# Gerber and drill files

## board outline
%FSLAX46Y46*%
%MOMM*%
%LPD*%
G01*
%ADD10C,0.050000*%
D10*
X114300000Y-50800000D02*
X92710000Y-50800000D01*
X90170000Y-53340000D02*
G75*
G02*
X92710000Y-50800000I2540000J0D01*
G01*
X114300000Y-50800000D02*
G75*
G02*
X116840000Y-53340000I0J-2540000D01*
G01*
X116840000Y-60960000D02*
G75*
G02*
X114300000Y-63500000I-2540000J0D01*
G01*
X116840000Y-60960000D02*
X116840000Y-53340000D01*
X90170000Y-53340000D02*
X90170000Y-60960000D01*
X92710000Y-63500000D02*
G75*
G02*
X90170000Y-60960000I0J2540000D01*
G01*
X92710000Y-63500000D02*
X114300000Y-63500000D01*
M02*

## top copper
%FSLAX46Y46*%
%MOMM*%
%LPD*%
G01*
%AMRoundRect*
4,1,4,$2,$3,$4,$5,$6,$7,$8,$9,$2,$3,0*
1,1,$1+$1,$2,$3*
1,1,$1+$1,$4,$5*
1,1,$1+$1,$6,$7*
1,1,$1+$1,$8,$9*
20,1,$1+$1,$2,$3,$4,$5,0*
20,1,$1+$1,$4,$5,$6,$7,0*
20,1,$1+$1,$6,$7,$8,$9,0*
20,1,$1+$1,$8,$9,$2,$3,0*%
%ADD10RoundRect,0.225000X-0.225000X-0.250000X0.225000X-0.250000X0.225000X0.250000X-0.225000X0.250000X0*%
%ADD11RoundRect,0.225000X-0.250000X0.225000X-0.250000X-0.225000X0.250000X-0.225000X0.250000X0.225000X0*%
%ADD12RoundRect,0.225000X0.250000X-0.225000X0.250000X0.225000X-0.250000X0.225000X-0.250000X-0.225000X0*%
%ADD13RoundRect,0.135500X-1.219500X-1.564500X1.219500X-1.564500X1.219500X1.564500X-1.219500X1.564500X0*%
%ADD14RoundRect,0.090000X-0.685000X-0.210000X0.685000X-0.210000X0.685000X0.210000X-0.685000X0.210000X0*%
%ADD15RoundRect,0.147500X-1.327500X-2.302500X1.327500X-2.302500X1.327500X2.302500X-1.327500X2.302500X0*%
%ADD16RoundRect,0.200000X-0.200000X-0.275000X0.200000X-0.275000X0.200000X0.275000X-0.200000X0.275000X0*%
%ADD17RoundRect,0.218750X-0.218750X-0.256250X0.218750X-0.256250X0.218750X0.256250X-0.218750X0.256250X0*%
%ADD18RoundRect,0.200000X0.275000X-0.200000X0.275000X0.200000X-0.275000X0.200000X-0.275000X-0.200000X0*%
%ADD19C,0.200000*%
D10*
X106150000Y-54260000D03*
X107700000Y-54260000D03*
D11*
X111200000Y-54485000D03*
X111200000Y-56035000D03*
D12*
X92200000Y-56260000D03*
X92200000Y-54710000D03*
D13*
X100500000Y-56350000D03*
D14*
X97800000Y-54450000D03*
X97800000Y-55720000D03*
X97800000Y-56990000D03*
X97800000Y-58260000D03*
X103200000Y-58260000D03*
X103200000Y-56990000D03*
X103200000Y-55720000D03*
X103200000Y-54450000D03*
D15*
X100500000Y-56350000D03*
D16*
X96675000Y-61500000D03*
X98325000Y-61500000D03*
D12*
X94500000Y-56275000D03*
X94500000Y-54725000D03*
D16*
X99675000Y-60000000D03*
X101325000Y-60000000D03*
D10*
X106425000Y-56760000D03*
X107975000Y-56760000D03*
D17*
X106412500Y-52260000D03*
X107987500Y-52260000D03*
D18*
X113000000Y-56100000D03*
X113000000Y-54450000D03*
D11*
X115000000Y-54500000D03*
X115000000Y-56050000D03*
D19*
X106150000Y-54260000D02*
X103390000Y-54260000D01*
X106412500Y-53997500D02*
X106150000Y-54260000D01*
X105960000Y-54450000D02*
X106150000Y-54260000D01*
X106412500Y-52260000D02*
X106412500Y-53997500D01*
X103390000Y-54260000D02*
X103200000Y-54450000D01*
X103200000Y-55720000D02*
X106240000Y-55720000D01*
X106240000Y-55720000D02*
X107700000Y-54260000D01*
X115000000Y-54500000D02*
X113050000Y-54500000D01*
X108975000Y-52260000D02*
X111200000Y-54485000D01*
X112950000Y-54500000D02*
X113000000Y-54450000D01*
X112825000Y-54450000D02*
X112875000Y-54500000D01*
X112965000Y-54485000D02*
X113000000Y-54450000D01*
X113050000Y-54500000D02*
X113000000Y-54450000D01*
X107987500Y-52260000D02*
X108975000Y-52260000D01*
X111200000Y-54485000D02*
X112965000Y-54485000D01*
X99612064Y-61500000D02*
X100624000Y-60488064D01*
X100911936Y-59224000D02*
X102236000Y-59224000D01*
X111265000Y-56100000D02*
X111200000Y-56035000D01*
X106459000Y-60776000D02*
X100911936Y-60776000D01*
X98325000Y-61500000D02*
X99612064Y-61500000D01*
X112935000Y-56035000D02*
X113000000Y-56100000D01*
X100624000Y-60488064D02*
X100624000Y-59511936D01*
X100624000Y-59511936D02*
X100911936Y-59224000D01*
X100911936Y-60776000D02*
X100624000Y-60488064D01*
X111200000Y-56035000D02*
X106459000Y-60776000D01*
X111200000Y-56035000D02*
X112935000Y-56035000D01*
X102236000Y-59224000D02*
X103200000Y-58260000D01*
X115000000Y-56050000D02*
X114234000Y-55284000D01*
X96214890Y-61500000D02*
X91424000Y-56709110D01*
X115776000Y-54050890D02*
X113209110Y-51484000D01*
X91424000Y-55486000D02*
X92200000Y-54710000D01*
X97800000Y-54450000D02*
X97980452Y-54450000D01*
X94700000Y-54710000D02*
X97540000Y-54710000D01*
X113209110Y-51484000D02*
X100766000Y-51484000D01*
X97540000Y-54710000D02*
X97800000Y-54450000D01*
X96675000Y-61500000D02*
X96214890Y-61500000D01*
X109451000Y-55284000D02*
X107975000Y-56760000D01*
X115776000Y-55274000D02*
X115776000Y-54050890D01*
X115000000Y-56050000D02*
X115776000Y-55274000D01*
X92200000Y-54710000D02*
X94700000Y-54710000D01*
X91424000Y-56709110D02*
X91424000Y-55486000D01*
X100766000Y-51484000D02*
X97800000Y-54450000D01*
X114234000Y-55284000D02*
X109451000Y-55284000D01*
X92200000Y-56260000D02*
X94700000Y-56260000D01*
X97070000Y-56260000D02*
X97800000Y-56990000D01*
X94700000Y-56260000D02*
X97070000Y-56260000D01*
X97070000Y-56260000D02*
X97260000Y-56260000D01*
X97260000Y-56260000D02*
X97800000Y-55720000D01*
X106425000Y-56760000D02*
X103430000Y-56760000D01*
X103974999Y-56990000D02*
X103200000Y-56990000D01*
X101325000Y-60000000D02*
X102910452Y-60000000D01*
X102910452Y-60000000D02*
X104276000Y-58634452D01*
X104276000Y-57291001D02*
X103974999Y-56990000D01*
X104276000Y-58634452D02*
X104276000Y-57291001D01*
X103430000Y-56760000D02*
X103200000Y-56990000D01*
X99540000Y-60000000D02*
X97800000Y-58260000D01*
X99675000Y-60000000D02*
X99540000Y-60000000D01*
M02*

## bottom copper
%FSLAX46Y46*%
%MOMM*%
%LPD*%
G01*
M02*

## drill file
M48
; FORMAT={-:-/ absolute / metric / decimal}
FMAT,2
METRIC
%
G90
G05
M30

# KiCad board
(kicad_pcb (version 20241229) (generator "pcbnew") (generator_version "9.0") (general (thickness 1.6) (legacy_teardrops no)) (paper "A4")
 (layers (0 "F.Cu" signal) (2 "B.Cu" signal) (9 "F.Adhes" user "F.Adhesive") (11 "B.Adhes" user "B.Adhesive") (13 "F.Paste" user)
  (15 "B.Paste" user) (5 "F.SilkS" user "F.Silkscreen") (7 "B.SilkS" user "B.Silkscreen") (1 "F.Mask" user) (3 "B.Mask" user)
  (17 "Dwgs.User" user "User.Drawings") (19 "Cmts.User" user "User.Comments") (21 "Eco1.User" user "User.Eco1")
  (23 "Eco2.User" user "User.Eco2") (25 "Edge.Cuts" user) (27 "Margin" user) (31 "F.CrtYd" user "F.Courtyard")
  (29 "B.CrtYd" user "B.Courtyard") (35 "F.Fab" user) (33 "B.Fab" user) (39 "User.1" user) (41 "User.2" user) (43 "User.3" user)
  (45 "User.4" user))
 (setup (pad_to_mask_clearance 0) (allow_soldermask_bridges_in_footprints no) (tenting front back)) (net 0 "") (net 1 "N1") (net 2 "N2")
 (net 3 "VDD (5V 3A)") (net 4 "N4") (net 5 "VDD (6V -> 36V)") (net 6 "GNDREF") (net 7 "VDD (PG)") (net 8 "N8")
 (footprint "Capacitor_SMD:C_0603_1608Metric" (layer "F.Cu") (at 106.925 54.26)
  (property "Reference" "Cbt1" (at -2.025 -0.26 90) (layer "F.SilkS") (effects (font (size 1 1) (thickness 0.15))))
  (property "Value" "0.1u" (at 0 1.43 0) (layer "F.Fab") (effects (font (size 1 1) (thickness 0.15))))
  (pad "1" smd roundrect (at -0.775 0) (size 0.9 0.95) (layers "F.Cu" "F.Mask" "F.Paste") (roundrect_rratio 0.25) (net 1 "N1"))
  (pad "2" smd roundrect (at 0.775 0) (size 0.9 0.95) (layers "F.Cu" "F.Mask" "F.Paste") (roundrect_rratio 0.25) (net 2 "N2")))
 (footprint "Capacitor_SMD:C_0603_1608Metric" (layer "F.Cu") (at 111.2 55.26 -90)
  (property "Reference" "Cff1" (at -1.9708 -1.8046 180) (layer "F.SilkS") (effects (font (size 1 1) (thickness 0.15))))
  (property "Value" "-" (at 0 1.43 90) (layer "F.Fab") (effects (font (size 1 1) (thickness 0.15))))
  (pad "1" smd roundrect (at -0.775 0 270) (size 0.9 0.95) (layers "F.Cu" "F.Mask" "F.Paste") (roundrect_rratio 0.25) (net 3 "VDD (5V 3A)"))
  (pad "2" smd roundrect (at 0.775 0 270) (size 0.9 0.95) (layers "F.Cu" "F.Mask" "F.Paste") (roundrect_rratio 0.25) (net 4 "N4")))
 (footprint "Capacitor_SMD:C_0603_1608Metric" (layer "F.Cu") (at 92.2 55.485 90)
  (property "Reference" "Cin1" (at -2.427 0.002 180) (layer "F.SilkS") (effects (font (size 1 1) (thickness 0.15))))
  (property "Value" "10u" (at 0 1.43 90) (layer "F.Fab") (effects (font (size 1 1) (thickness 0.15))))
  (pad "1" smd roundrect (at -0.775 0 90) (size 0.9 0.95) (layers "F.Cu" "F.Mask" "F.Paste") (roundrect_rratio 0.25)
   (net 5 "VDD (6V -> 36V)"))
  (pad "2" smd roundrect (at 0.775 0 90) (size 0.9 0.95) (layers "F.Cu" "F.Mask" "F.Paste") (roundrect_rratio 0.25) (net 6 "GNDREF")))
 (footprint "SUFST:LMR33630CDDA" (layer "F.Cu") (at 100.4 53.35)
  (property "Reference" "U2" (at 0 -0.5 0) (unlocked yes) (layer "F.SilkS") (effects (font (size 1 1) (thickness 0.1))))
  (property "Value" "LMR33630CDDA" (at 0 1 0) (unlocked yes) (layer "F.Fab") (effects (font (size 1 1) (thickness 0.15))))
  (pad "" smd roundrect (at 0.1 3) (size 2.71 3.4) (layers "F.Cu" "F.Mask" "F.Paste") (roundrect_rratio 0.05))
  (pad "1" smd roundrect (at -2.6 1.1) (size 1.55 0.6) (layers "F.Cu" "F.Mask" "F.Paste") (roundrect_rratio 0.15) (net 6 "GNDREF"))
  (pad "2" smd roundrect (at -2.6 2.37) (size 1.55 0.6) (layers "F.Cu" "F.Mask" "F.Paste") (roundrect_rratio 0.15) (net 5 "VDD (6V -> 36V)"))
  (pad "3" smd roundrect (at -2.6 3.64) (size 1.55 0.6) (layers "F.Cu" "F.Mask" "F.Paste") (roundrect_rratio 0.15) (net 5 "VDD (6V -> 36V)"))
  (pad "4" smd roundrect (at -2.6 4.91) (size 1.55 0.6) (layers "F.Cu" "F.Mask" "F.Paste") (roundrect_rratio 0.15) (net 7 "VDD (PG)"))
  (pad "5" smd roundrect (at 2.8 4.91) (size 1.55 0.6) (layers "F.Cu" "F.Mask" "F.Paste") (roundrect_rratio 0.15) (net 4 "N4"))
  (pad "6" smd roundrect (at 2.8 3.64) (size 1.55 0.6) (layers "F.Cu" "F.Mask" "F.Paste") (roundrect_rratio 0.15) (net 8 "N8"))
  (pad "7" smd roundrect (at 2.8 2.37) (size 1.55 0.6) (layers "F.Cu" "F.Mask" "F.Paste") (roundrect_rratio 0.15) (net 2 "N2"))
  (pad "8" smd roundrect (at 2.8 1.1) (size 1.55 0.6) (layers "F.Cu" "F.Mask" "F.Paste") (roundrect_rratio 0.15) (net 1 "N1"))
  (pad "TP" smd roundrect (at 0.1 3) (size 2.95 4.9) (layers "F.Cu") (roundrect_rratio 0.05) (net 6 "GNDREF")))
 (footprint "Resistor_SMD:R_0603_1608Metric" (layer "F.Cu") (at 97.5 61.5)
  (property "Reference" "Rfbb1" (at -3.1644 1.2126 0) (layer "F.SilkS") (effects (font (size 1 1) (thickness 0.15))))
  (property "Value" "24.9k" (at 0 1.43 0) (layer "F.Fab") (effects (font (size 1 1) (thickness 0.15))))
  (pad "1" smd roundrect (at -0.825 0) (size 0.8 0.95) (layers "F.Cu" "F.Mask" "F.Paste") (roundrect_rratio 0.25) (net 6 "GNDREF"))
  (pad "2" smd roundrect (at 0.825 0) (size 0.8 0.95) (layers "F.Cu" "F.Mask" "F.Paste") (roundrect_rratio 0.25) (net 4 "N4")))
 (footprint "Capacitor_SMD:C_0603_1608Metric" (layer "F.Cu") (at 94.5 55.5 90)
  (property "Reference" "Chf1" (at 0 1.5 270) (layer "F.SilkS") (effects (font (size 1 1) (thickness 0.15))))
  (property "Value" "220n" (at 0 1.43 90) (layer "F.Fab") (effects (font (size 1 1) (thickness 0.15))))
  (pad "1" smd roundrect (at -0.775 0 90) (size 0.9 0.95) (layers "F.Cu" "F.Mask" "F.Paste") (roundrect_rratio 0.25)
   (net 5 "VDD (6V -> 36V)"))
  (pad "2" smd roundrect (at 0.775 0 90) (size 0.9 0.95) (layers "F.Cu" "F.Mask" "F.Paste") (roundrect_rratio 0.25) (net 6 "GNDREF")))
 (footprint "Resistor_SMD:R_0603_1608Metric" (layer "F.Cu") (at 100.5 60)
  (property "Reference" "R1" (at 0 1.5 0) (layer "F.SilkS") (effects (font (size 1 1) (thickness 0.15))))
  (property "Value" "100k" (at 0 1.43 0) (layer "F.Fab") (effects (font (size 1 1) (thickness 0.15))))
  (pad "1" smd roundrect (at -0.825 0) (size 0.8 0.95) (layers "F.Cu" "F.Mask" "F.Paste") (roundrect_rratio 0.25) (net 7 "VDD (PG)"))
  (pad "2" smd roundrect (at 0.825 0) (size 0.8 0.95) (layers "F.Cu" "F.Mask" "F.Paste") (roundrect_rratio 0.25) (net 8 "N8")))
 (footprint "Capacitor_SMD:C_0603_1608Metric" (layer "F.Cu") (at 107.2 56.76)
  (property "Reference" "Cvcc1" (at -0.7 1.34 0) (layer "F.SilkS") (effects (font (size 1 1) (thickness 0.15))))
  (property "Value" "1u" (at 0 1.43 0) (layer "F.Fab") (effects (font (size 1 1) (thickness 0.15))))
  (pad "1" smd roundrect (at -0.775 0) (size 0.9 0.95) (layers "F.Cu" "F.Mask" "F.Paste") (roundrect_rratio 0.25) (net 8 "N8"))
  (pad "2" smd roundrect (at 0.775 0) (size 0.9 0.95) (layers "F.Cu" "F.Mask" "F.Paste") (roundrect_rratio 0.25) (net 6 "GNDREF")))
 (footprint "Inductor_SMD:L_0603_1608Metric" (layer "F.Cu") (at 107.2 52.26)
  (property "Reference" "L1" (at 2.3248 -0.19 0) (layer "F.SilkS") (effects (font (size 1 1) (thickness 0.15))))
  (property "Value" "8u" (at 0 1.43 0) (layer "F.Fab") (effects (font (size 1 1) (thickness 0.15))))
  (pad "1" smd roundrect (at -0.7875 0) (size 0.875 0.95) (layers "F.Cu" "F.Mask" "F.Paste") (roundrect_rratio 0.25) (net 1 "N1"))
  (pad "2" smd roundrect (at 0.7875 0) (size 0.875 0.95) (layers "F.Cu" "F.Mask" "F.Paste") (roundrect_rratio 0.25) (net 3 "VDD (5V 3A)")))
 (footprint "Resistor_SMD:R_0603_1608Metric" (layer "F.Cu") (at 113 55.275 90)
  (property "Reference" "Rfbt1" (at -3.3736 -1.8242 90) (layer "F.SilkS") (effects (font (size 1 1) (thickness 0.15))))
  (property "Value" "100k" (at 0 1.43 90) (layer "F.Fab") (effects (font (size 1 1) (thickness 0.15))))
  (pad "1" smd roundrect (at -0.825 0 90) (size 0.8 0.95) (layers "F.Cu" "F.Mask" "F.Paste") (roundrect_rratio 0.25) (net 4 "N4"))
  (pad "2" smd roundrect (at 0.825 0 90) (size 0.8 0.95) (layers "F.Cu" "F.Mask" "F.Paste") (roundrect_rratio 0.25) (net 3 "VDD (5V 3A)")))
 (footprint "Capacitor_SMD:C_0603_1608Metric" (layer "F.Cu") (at 115 55.275 -90)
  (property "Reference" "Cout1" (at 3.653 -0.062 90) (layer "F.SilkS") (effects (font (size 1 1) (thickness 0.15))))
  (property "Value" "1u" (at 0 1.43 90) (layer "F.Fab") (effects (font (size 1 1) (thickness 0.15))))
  (pad "1" smd roundrect (at -0.775 0 270) (size 0.9 0.95) (layers "F.Cu" "F.Mask" "F.Paste") (roundrect_rratio 0.25) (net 3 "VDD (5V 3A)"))
  (pad "2" smd roundrect (at 0.775 0 270) (size 0.9 0.95) (layers "F.Cu" "F.Mask" "F.Paste") (roundrect_rratio 0.25) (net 6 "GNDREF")))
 (gr_line (start 114.3 50.8) (end 92.71 50.8) (stroke (width 0.05) (type default)) (layer "Edge.Cuts"))
 (gr_arc (start 90.17 53.34) (mid 90.913949 51.543949) (end 92.71 50.8) (stroke (width 0.05) (type default)) (layer "Edge.Cuts"))
 (gr_arc (start 114.3 50.8) (mid 116.096051 51.543949) (end 116.84 53.34) (stroke (width 0.05) (type default)) (layer "Edge.Cuts"))
 (gr_arc (start 116.84 60.96) (mid 116.096051 62.756051) (end 114.3 63.5) (stroke (width 0.05) (type default)) (layer "Edge.Cuts"))
 (gr_line (start 116.84 60.96) (end 116.84 53.34) (stroke (width 0.05) (type default)) (layer "Edge.Cuts"))
 (gr_line (start 90.17 53.34) (end 90.17 60.96) (stroke (width 0.05) (type default)) (layer "Edge.Cuts"))
 (gr_arc (start 92.71 63.5) (mid 90.913949 62.756051) (end 90.17 60.96) (stroke (width 0.05) (type default)) (layer "Edge.Cuts"))
 (gr_line (start 92.71 63.5) (end 114.3 63.5) (stroke (width 0.05) (type default)) (layer "Edge.Cuts"))
 (segment (start 106.15 54.26) (end 103.39 54.26) (width 0.2) (layer "F.Cu") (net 1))
 (segment (start 106.4125 53.9975) (end 106.15 54.26) (width 0.2) (layer "F.Cu") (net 1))
 (segment (start 105.96 54.45) (end 106.15 54.26) (width 0.2) (layer "F.Cu") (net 1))
 (segment (start 106.4125 52.26) (end 106.4125 53.9975) (width 0.2) (layer "F.Cu") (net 1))
 (segment (start 103.39 54.26) (end 103.2 54.45) (width 0.2) (layer "F.Cu") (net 1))
 (segment (start 103.2 55.72) (end 106.24 55.72) (width 0.2) (layer "F.Cu") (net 2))
 (segment (start 106.24 55.72) (end 107.7 54.26) (width 0.2) (layer "F.Cu") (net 2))
 (segment (start 115 54.5) (end 113.05 54.5) (width 0.2) (layer "F.Cu") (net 3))
 (segment (start 108.975 52.26) (end 111.2 54.485) (width 0.2) (layer "F.Cu") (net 3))
 (segment (start 112.95 54.5) (end 113 54.45) (width 0.2) (layer "F.Cu") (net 3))
 (segment (start 112.825 54.45) (end 112.875 54.5) (width 0.2) (layer "F.Cu") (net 3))
 (segment (start 112.965 54.485) (end 113 54.45) (width 0.2) (layer "F.Cu") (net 3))
 (segment (start 113.05 54.5) (end 113 54.45) (width 0.2) (layer "F.Cu") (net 3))
 (segment (start 107.9875 52.26) (end 108.975 52.26) (width 0.2) (layer "F.Cu") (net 3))
 (segment (start 111.2 54.485) (end 112.965 54.485) (width 0.2) (layer "F.Cu") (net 3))
 (segment (start 99.612064 61.5) (end 100.624 60.488064) (width 0.2) (layer "F.Cu") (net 4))
 (segment (start 100.911936 59.224) (end 102.236 59.224) (width 0.2) (layer "F.Cu") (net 4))
 (segment (start 111.265 56.1) (end 111.2 56.035) (width 0.2) (layer "F.Cu") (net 4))
 (segment (start 106.459 60.776) (end 100.911936 60.776) (width 0.2) (layer "F.Cu") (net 4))
 (segment (start 98.325 61.5) (end 99.612064 61.5) (width 0.2) (layer "F.Cu") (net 4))
 (segment (start 112.935 56.035) (end 113 56.1) (width 0.2) (layer "F.Cu") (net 4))
 (segment (start 100.624 60.488064) (end 100.624 59.511936) (width 0.2) (layer "F.Cu") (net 4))
 (segment (start 100.624 59.511936) (end 100.911936 59.224) (width 0.2) (layer "F.Cu") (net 4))
 (segment (start 100.911936 60.776) (end 100.624 60.488064) (width 0.2) (layer "F.Cu") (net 4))
 (segment (start 111.2 56.035) (end 106.459 60.776) (width 0.2) (layer "F.Cu") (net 4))
 (segment (start 111.2 56.035) (end 112.935 56.035) (width 0.2) (layer "F.Cu") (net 4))
 (segment (start 102.236 59.224) (end 103.2 58.26) (width 0.2) (layer "F.Cu") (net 4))
 (segment (start 115 56.05) (end 114.234 55.284) (width 0.2) (layer "F.Cu") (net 6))
 (segment (start 96.21489 61.5) (end 91.424 56.70911) (width 0.2) (layer "F.Cu") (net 6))
 (segment (start 115.776 54.05089) (end 113.20911 51.484) (width 0.2) (layer "F.Cu") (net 6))
 (segment (start 91.424 55.486) (end 92.2 54.71) (width 0.2) (layer "F.Cu") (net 6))
 (segment (start 97.8 54.45) (end 97.980452 54.45) (width 0.2) (layer "F.Cu") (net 6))
 (segment (start 94.7 54.71) (end 97.54 54.71) (width 0.2) (layer "F.Cu") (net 6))
 (segment (start 113.20911 51.484) (end 100.766 51.484) (width 0.2) (layer "F.Cu") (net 6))
 (segment (start 97.54 54.71) (end 97.8 54.45) (width 0.2) (layer "F.Cu") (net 6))
 (segment (start 96.675 61.5) (end 96.21489 61.5) (width 0.2) (layer "F.Cu") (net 6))
 (segment (start 109.451 55.284) (end 107.975 56.76) (width 0.2) (layer "F.Cu") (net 6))
 (segment (start 115.776 55.274) (end 115.776 54.05089) (width 0.2) (layer "F.Cu") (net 6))
 (segment (start 115 56.05) (end 115.776 55.274) (width 0.2) (layer "F.Cu") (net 6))
 (segment (start 92.2 54.71) (end 94.7 54.71) (width 0.2) (layer "F.Cu") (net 6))
 (segment (start 91.424 56.70911) (end 91.424 55.486) (width 0.2) (layer "F.Cu") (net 6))
 (segment (start 100.766 51.484) (end 97.8 54.45) (width 0.2) (layer "F.Cu") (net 6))
 (segment (start 114.234 55.284) (end 109.451 55.284) (width 0.2) (layer "F.Cu") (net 6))
 (segment (start 92.2 56.26) (end 94.7 56.26) (width 0.2) (layer "F.Cu") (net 5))
 (segment (start 97.07 56.26) (end 97.8 56.99) (width 0.2) (layer "F.Cu") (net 5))
 (segment (start 94.7 56.26) (end 97.07 56.26) (width 0.2) (layer "F.Cu") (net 5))
 (segment (start 97.07 56.26) (end 97.26 56.26) (width 0.2) (layer "F.Cu") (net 5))
 (segment (start 97.26 56.26) (end 97.8 55.72) (width 0.2) (layer "F.Cu") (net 5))
 (segment (start 106.425 56.76) (end 103.43 56.76) (width 0.2) (layer "F.Cu") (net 8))
 (segment (start 103.974999 56.99) (end 103.2 56.99) (width 0.2) (layer "F.Cu") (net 8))
 (segment (start 101.325 60) (end 102.910452 60) (width 0.2) (layer "F.Cu") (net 8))
 (segment (start 102.910452 60) (end 104.276 58.634452) (width 0.2) (layer "F.Cu") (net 8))
 (segment (start 104.276 57.291001) (end 103.974999 56.99) (width 0.2) (layer "F.Cu") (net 8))
 (segment (start 104.276 58.634452) (end 104.276 57.291001) (width 0.2) (layer "F.Cu") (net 8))
 (segment (start 103.43 56.76) (end 103.2 56.99) (width 0.2) (layer "F.Cu") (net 8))
 (segment (start 99.54 60) (end 97.8 58.26) (width 0.2) (layer "F.Cu") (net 7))
 (segment (start 99.675 60) (end 99.54 60) (width 0.2) (layer "F.Cu") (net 7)))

